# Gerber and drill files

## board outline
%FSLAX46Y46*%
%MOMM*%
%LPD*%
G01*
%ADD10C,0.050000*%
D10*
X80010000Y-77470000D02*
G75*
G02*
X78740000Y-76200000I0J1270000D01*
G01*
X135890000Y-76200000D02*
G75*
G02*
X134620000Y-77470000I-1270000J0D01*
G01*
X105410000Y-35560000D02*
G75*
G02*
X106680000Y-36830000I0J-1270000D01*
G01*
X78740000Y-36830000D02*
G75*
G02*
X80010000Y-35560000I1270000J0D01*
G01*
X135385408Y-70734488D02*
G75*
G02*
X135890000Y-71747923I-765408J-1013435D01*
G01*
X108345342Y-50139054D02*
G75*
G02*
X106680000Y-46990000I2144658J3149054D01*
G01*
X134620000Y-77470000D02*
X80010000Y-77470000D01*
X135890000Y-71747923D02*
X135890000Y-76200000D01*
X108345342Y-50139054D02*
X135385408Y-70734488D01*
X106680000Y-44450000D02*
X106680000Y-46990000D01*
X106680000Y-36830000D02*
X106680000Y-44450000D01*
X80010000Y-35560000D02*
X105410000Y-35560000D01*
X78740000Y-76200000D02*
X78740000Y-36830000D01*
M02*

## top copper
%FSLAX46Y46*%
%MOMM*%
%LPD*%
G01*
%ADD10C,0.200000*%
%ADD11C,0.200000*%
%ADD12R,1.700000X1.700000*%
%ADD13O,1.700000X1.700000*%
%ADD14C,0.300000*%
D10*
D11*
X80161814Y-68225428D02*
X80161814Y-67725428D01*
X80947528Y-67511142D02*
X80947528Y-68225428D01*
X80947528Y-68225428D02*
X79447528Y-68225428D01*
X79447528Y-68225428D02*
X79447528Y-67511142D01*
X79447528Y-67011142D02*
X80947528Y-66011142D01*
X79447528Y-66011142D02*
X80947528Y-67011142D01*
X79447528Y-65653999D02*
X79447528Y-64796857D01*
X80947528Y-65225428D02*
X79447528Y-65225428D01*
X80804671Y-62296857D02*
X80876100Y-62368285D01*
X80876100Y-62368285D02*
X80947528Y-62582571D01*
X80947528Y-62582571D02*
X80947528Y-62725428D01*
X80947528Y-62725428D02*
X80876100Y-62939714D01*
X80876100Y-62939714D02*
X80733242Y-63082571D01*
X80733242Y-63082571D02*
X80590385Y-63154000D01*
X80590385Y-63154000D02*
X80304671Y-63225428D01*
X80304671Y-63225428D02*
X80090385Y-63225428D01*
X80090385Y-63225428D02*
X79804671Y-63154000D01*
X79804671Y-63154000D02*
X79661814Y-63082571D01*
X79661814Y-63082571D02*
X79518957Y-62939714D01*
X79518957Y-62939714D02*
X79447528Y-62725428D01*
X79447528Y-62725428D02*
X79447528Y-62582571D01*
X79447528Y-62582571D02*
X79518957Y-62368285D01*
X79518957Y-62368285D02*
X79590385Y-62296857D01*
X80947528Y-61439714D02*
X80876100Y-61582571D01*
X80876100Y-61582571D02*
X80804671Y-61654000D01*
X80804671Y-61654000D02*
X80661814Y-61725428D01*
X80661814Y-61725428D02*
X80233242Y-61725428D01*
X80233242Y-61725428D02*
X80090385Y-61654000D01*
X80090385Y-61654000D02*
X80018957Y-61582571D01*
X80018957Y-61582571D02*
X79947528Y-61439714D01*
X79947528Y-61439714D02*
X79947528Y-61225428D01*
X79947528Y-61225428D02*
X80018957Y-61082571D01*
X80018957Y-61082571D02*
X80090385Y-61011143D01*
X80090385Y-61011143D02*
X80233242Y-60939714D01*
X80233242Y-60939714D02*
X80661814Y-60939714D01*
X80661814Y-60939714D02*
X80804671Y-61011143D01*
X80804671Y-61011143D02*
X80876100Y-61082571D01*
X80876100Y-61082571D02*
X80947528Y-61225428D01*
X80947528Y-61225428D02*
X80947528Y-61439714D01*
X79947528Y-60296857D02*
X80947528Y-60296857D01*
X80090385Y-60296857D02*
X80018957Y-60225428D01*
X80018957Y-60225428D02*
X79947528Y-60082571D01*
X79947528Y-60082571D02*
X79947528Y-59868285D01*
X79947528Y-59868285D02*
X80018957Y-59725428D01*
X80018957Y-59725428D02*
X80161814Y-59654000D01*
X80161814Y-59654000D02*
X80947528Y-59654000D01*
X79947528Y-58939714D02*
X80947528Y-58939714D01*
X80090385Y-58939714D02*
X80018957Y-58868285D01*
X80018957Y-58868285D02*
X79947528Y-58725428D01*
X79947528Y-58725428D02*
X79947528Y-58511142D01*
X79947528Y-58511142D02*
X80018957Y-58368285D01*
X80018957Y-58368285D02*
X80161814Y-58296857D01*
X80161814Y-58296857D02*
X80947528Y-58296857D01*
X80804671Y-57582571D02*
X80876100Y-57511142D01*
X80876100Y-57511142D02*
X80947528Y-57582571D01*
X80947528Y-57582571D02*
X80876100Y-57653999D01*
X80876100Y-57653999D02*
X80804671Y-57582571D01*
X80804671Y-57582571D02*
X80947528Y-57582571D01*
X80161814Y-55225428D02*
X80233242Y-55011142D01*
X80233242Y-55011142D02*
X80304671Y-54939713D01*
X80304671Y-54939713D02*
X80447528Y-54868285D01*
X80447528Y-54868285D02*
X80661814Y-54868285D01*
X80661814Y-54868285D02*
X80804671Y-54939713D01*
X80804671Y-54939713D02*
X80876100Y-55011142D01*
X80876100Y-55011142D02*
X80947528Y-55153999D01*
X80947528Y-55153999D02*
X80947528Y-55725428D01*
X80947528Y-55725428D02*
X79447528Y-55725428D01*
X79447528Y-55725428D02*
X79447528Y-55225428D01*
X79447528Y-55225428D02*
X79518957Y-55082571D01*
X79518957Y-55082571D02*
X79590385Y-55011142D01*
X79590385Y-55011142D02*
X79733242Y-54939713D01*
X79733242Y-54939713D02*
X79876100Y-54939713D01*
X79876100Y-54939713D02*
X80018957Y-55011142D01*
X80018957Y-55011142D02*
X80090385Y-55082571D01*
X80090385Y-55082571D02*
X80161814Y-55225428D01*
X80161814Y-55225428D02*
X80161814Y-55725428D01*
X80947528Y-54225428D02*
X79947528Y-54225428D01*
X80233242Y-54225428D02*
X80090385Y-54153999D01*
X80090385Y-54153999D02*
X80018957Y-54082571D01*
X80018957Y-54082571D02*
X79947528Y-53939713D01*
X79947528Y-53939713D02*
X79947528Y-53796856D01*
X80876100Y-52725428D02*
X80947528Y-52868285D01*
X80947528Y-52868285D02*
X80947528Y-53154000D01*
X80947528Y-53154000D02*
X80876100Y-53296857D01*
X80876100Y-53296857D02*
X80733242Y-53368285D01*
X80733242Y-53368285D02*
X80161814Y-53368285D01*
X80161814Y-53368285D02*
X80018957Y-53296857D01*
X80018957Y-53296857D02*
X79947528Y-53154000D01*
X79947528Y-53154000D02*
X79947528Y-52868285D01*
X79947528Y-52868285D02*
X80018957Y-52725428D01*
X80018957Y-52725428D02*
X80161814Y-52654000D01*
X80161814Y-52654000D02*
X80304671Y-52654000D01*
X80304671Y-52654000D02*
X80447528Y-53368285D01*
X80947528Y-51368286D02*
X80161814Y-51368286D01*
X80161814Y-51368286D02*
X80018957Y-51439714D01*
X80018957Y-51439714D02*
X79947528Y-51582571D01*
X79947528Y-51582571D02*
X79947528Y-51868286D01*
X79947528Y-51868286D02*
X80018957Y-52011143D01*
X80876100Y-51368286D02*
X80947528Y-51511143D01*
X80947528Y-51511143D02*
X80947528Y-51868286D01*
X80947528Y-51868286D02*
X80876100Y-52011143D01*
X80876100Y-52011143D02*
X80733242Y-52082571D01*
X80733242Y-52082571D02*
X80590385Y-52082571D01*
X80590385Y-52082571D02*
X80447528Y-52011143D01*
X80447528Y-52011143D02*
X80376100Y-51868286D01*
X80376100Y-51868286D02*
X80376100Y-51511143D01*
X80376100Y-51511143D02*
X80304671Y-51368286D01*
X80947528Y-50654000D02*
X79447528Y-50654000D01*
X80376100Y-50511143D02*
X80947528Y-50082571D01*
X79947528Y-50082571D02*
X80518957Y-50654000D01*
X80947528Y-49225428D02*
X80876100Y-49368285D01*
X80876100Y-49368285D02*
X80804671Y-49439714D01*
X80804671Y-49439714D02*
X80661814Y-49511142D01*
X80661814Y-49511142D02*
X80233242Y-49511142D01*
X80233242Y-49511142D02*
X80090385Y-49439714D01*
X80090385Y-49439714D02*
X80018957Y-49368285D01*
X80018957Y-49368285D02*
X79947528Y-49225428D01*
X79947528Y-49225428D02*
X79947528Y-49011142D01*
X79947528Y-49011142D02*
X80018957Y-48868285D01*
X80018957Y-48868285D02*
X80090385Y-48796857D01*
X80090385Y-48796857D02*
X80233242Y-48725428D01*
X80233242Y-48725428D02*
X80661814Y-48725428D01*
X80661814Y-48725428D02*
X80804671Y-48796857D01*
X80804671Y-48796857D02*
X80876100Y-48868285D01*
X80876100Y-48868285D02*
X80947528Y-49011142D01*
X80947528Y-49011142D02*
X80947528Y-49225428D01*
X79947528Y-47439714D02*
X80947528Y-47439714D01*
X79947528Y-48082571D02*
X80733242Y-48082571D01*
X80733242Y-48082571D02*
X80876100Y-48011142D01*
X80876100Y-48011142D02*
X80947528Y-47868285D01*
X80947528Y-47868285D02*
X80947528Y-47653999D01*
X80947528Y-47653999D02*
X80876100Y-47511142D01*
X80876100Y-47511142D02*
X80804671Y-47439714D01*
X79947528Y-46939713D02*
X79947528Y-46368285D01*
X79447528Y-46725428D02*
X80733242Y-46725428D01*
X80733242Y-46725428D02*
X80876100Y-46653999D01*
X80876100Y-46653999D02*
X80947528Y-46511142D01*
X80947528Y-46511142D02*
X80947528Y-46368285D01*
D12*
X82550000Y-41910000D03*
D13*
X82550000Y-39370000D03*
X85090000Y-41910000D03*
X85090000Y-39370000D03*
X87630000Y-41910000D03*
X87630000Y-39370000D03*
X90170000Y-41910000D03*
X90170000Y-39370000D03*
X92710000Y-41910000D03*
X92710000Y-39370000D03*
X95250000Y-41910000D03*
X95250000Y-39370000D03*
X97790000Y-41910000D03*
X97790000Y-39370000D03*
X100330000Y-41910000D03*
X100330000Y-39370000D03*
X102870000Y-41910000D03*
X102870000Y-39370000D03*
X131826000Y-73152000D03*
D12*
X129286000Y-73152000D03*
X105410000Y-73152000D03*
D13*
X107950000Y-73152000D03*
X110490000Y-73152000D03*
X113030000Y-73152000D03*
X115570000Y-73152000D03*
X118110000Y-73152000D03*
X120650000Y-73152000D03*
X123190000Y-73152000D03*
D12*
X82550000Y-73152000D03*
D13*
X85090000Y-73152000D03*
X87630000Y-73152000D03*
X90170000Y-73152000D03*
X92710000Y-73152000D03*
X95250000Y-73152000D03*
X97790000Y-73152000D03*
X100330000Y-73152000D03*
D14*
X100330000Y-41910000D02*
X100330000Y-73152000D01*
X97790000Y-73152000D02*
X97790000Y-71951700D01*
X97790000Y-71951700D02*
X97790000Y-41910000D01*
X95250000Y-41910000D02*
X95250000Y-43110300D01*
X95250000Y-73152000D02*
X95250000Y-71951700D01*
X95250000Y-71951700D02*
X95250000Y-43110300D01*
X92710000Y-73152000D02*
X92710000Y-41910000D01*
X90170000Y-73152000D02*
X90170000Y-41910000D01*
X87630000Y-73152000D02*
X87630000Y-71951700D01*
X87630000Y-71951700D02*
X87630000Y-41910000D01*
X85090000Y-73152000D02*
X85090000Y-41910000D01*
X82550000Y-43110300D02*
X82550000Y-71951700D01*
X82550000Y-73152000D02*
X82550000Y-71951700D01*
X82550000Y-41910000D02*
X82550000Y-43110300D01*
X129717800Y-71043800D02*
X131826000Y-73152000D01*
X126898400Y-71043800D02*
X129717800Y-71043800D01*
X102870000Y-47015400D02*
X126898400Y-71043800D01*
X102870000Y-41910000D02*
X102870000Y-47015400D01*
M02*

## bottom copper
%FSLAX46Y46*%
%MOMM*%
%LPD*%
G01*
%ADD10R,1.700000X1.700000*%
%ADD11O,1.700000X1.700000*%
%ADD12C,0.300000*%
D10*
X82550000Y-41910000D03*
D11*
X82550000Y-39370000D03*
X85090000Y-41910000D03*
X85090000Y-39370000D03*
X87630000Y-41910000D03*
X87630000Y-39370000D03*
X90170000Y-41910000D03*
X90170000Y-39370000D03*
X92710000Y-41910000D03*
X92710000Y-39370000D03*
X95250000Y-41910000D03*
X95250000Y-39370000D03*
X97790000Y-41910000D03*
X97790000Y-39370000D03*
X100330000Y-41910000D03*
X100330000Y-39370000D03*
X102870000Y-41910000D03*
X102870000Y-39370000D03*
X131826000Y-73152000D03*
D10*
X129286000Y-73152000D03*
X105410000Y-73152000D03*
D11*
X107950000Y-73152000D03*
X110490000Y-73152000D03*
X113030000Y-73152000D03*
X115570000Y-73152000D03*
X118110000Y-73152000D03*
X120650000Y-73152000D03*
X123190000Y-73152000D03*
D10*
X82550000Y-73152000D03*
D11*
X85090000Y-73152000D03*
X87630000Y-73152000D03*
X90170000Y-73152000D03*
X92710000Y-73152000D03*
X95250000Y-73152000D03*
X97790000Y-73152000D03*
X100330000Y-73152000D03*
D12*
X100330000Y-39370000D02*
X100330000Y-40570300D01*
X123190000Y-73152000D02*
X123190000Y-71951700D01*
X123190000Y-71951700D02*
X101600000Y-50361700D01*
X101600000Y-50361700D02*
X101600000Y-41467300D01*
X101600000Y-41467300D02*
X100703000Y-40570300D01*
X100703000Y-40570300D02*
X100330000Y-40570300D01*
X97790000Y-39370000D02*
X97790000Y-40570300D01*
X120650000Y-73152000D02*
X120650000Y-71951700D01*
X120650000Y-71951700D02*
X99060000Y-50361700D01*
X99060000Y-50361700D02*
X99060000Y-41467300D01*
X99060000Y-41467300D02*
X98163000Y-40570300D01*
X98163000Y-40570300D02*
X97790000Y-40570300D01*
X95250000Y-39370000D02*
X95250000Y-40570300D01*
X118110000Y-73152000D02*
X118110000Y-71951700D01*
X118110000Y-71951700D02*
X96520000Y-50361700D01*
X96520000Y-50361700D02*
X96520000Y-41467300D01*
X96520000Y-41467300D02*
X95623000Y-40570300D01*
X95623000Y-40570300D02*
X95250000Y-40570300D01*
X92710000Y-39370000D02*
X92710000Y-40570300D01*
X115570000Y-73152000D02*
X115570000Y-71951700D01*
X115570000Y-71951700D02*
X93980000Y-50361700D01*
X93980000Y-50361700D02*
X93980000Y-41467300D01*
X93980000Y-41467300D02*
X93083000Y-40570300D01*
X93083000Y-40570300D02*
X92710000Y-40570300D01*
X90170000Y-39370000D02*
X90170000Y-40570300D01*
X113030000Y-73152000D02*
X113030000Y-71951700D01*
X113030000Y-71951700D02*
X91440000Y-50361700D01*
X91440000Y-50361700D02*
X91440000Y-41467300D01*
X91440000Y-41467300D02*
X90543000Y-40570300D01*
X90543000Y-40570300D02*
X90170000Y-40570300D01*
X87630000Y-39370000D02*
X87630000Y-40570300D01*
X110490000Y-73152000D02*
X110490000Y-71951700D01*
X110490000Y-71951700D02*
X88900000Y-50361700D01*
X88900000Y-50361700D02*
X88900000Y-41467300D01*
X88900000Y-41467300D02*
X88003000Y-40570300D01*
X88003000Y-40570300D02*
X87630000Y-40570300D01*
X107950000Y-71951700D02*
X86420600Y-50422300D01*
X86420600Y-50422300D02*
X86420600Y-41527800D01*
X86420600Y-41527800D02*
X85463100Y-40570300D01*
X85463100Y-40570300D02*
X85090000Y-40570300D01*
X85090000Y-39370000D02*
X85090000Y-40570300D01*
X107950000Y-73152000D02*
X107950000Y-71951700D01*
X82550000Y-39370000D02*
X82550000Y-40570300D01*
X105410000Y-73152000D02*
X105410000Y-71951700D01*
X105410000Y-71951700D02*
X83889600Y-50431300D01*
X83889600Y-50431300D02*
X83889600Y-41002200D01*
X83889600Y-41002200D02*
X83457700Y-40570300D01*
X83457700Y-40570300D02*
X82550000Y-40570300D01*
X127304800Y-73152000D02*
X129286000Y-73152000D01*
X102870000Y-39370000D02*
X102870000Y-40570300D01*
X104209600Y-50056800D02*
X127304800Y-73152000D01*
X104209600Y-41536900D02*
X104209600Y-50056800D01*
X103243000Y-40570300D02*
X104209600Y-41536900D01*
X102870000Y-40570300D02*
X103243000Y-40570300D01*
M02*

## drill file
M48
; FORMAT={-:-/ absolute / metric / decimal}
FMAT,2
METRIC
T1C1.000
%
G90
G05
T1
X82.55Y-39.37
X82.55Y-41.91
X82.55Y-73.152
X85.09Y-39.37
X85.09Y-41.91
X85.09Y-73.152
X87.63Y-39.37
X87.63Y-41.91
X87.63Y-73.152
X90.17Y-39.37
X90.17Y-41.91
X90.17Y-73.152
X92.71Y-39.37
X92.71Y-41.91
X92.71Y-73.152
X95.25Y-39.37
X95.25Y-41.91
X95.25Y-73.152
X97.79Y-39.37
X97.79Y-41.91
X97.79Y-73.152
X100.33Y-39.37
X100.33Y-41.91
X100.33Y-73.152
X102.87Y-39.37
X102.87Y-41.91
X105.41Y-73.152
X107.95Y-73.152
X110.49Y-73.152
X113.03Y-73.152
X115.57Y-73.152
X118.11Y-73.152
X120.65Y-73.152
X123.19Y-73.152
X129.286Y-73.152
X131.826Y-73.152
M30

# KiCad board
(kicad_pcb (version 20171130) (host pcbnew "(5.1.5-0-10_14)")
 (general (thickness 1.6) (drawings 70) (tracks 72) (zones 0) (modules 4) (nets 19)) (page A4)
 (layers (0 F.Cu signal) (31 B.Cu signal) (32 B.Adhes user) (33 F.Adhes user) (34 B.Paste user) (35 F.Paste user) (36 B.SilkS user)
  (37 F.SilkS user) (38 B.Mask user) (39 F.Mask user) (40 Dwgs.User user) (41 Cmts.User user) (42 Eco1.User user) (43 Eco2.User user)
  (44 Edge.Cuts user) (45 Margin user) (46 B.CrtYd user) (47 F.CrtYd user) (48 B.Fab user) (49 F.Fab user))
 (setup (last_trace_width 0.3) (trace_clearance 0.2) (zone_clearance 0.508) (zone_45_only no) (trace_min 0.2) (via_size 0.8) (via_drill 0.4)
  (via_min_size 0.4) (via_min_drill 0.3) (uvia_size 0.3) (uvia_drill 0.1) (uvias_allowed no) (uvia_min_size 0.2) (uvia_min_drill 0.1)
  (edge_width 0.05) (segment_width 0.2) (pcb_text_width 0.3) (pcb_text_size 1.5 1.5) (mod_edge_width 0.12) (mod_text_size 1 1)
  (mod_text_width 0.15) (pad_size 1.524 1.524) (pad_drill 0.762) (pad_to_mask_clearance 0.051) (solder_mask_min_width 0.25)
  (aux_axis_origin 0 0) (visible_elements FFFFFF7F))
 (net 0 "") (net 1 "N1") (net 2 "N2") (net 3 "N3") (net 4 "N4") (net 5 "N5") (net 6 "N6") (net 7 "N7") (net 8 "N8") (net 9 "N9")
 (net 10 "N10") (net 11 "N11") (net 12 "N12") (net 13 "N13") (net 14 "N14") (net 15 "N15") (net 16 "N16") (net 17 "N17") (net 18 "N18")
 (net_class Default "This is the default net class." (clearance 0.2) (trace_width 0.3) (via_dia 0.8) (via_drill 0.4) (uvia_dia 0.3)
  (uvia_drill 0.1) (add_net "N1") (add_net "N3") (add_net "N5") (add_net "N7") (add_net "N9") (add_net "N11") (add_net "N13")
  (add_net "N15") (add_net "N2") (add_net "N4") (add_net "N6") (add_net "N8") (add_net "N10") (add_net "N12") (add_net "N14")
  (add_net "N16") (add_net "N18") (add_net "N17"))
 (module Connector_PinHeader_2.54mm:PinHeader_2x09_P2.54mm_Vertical (layer F.Cu) (at 82.55 41.91 90)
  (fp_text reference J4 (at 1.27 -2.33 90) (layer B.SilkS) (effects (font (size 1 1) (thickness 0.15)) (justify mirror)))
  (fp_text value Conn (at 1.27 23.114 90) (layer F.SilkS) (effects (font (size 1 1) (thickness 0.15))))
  (pad 1 thru_hole rect (at 0 0 90) (size 1.7 1.7) (drill 1) (layers *.Cu *.Mask) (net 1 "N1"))
  (pad 2 thru_hole oval (at 2.54 0 90) (size 1.7 1.7) (drill 1) (layers *.Cu *.Mask) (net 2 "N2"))
  (pad 3 thru_hole oval (at 0 2.54 90) (size 1.7 1.7) (drill 1) (layers *.Cu *.Mask) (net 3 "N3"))
  (pad 4 thru_hole oval (at 2.54 2.54 90) (size 1.7 1.7) (drill 1) (layers *.Cu *.Mask) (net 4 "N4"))
  (pad 5 thru_hole oval (at 0 5.08 90) (size 1.7 1.7) (drill 1) (layers *.Cu *.Mask) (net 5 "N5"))
  (pad 6 thru_hole oval (at 2.54 5.08 90) (size 1.7 1.7) (drill 1) (layers *.Cu *.Mask) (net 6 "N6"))
  (pad 7 thru_hole oval (at 0 7.62 90) (size 1.7 1.7) (drill 1) (layers *.Cu *.Mask) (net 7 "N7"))
  (pad 8 thru_hole oval (at 2.54 7.62 90) (size 1.7 1.7) (drill 1) (layers *.Cu *.Mask) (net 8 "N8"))
  (pad 9 thru_hole oval (at 0 10.16 90) (size 1.7 1.7) (drill 1) (layers *.Cu *.Mask) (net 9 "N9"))
  (pad 10 thru_hole oval (at 2.54 10.16 90) (size 1.7 1.7) (drill 1) (layers *.Cu *.Mask) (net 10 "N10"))
  (pad 11 thru_hole oval (at 0 12.7 90) (size 1.7 1.7) (drill 1) (layers *.Cu *.Mask) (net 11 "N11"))
  (pad 12 thru_hole oval (at 2.54 12.7 90) (size 1.7 1.7) (drill 1) (layers *.Cu *.Mask) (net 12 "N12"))
  (pad 13 thru_hole oval (at 0 15.24 90) (size 1.7 1.7) (drill 1) (layers *.Cu *.Mask) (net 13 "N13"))
  (pad 14 thru_hole oval (at 2.54 15.24 90) (size 1.7 1.7) (drill 1) (layers *.Cu *.Mask) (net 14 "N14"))
  (pad 15 thru_hole oval (at 0 17.78 90) (size 1.7 1.7) (drill 1) (layers *.Cu *.Mask) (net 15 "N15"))
  (pad 16 thru_hole oval (at 2.54 17.78 90) (size 1.7 1.7) (drill 1) (layers *.Cu *.Mask) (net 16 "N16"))
  (pad 17 thru_hole oval (at 0 20.32 90) (size 1.7 1.7) (drill 1) (layers *.Cu *.Mask) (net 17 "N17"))
  (pad 18 thru_hole oval (at 2.54 20.32 90) (size 1.7 1.7) (drill 1) (layers *.Cu *.Mask) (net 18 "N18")))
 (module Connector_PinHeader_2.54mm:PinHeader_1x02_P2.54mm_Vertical (layer B.Cu) (at 129.286 73.152 270)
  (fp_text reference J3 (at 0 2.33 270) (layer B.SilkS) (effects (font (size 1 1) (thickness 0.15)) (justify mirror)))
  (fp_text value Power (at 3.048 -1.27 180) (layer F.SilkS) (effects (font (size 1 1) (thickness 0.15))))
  (pad 2 thru_hole oval (at 0 -2.54 270) (size 1.7 1.7) (drill 1) (layers *.Cu *.Mask) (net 17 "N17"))
  (pad 1 thru_hole rect (at 0 0 270) (size 1.7 1.7) (drill 1) (layers *.Cu *.Mask) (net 18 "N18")))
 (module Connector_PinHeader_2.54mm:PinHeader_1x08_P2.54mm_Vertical (layer B.Cu) (at 105.41 73.152 270)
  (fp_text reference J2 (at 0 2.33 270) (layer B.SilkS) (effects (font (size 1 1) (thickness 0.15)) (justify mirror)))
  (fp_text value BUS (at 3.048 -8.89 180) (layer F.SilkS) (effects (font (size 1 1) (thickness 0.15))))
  (pad 1 thru_hole rect (at 0 0 270) (size 1.7 1.7) (drill 1) (layers *.Cu *.Mask) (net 2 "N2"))
  (pad 2 thru_hole oval (at 0 -2.54 270) (size 1.7 1.7) (drill 1) (layers *.Cu *.Mask) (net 4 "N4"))
  (pad 3 thru_hole oval (at 0 -5.08 270) (size 1.7 1.7) (drill 1) (layers *.Cu *.Mask) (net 6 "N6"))
  (pad 4 thru_hole oval (at 0 -7.62 270) (size 1.7 1.7) (drill 1) (layers *.Cu *.Mask) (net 8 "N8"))
  (pad 5 thru_hole oval (at 0 -10.16 270) (size 1.7 1.7) (drill 1) (layers *.Cu *.Mask) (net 10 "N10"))
  (pad 6 thru_hole oval (at 0 -12.7 270) (size 1.7 1.7) (drill 1) (layers *.Cu *.Mask) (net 12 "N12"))
  (pad 7 thru_hole oval (at 0 -15.24 270) (size 1.7 1.7) (drill 1) (layers *.Cu *.Mask) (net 14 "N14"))
  (pad 8 thru_hole oval (at 0 -17.78 270) (size 1.7 1.7) (drill 1) (layers *.Cu *.Mask) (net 16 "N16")))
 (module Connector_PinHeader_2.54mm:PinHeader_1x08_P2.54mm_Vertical (layer B.Cu) (at 82.55 73.152 270)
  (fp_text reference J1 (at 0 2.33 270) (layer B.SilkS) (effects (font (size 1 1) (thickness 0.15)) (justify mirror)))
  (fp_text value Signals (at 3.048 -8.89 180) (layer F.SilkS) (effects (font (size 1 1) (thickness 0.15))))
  (pad 1 thru_hole rect (at 0 0 270) (size 1.7 1.7) (drill 1) (layers *.Cu *.Mask) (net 1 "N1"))
  (pad 2 thru_hole oval (at 0 -2.54 270) (size 1.7 1.7) (drill 1) (layers *.Cu *.Mask) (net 3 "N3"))
  (pad 3 thru_hole oval (at 0 -5.08 270) (size 1.7 1.7) (drill 1) (layers *.Cu *.Mask) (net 5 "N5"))
  (pad 4 thru_hole oval (at 0 -7.62 270) (size 1.7 1.7) (drill 1) (layers *.Cu *.Mask) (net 7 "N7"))
  (pad 5 thru_hole oval (at 0 -10.16 270) (size 1.7 1.7) (drill 1) (layers *.Cu *.Mask) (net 9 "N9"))
  (pad 6 thru_hole oval (at 0 -12.7 270) (size 1.7 1.7) (drill 1) (layers *.Cu *.Mask) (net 11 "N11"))
  (pad 7 thru_hole oval (at 0 -15.24 270) (size 1.7 1.7) (drill 1) (layers *.Cu *.Mask) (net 13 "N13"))
  (pad 8 thru_hole oval (at 0 -17.78 270) (size 1.7 1.7) (drill 1) (layers *.Cu *.Mask) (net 15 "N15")))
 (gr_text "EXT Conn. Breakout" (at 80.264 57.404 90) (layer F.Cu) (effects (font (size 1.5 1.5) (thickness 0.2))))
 (gr_arc (start 80.01 76.2) (end 78.74 76.2) (angle -90) (layer Edge.Cuts) (width 0.05))
 (gr_arc (start 134.62 76.2) (end 134.62 77.47) (angle -90) (layer Edge.Cuts) (width 0.05))
 (gr_arc (start 105.41 36.83) (end 106.68 36.83) (angle -90) (layer Edge.Cuts) (width 0.05))
 (gr_arc (start 80.01 36.83) (end 80.01 35.56) (angle -90) (layer Edge.Cuts) (width 0.05))
 (gr_arc (start 134.62 71.747923) (end 135.89 71.747923) (angle -52.93767885) (layer Edge.Cuts) (width 0.05))
 (gr_arc (start 110.49 46.99) (end 106.68 46.99) (angle -55.74323869) (layer Edge.Cuts) (width 0.05))
 (gr_line (start 134.62 77.47) (end 80.01 77.47) (layer Edge.Cuts) (width 0.05))
 (gr_line (start 135.89 71.747923) (end 135.89 76.2) (layer Edge.Cuts) (width 0.05))
 (gr_line (start 108.345342 50.139054) (end 135.385408 70.734488) (layer Edge.Cuts) (width 0.05))
 (gr_line (start 106.68 44.45) (end 106.68 46.99) (layer Edge.Cuts) (width 0.05))
 (gr_line (start 106.68 36.83) (end 106.68 44.45) (layer Edge.Cuts) (width 0.05))
 (gr_line (start 80.01 35.56) (end 105.41 35.56) (layer Edge.Cuts) (width 0.05))
 (gr_line (start 78.74 76.2) (end 78.74 36.83) (layer Edge.Cuts) (width 0.05))
 (segment (start 100.33 41.91) (end 100.33 73.152) (width 0.3) (layer F.Cu) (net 15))
 (segment (start 97.79 73.152) (end 97.79 71.9517) (width 0.3) (layer F.Cu) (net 13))
 (segment (start 97.79 71.9517) (end 97.79 41.91) (width 0.3) (layer F.Cu) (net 13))
 (segment (start 95.25 41.91) (end 95.25 43.1103) (width 0.3) (layer F.Cu) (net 11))
 (segment (start 95.25 73.152) (end 95.25 71.9517) (width 0.3) (layer F.Cu) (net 11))
 (segment (start 95.25 71.9517) (end 95.25 43.1103) (width 0.3) (layer F.Cu) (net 11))
 (segment (start 92.71 73.152) (end 92.71 41.91) (width 0.3) (layer F.Cu) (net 9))
 (segment (start 90.17 73.152) (end 90.17 41.91) (width 0.3) (layer F.Cu) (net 7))
 (segment (start 87.63 73.152) (end 87.63 71.9517) (width 0.3) (layer F.Cu) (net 5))
 (segment (start 87.63 71.9517) (end 87.63 41.91) (width 0.3) (layer F.Cu) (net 5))
 (segment (start 85.09 73.152) (end 85.09 41.91) (width 0.3) (layer F.Cu) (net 3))
 (segment (start 82.55 43.1103) (end 82.55 71.9517) (width 0.3) (layer F.Cu) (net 1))
 (segment (start 82.55 73.152) (end 82.55 71.9517) (width 0.3) (layer F.Cu) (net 1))
 (segment (start 82.55 41.91) (end 82.55 43.1103) (width 0.3) (layer F.Cu) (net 1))
 (segment (start 100.33 39.37) (end 100.33 40.5703) (width 0.3) (layer B.Cu) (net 16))
 (segment (start 123.19 73.152) (end 123.19 71.9517) (width 0.3) (layer B.Cu) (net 16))
 (segment (start 123.19 71.9517) (end 101.6 50.3617) (width 0.3) (layer B.Cu) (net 16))
 (segment (start 101.6 50.3617) (end 101.6 41.4673) (width 0.3) (layer B.Cu) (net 16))
 (segment (start 101.6 41.4673) (end 100.703 40.5703) (width 0.3) (layer B.Cu) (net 16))
 (segment (start 100.703 40.5703) (end 100.33 40.5703) (width 0.3) (layer B.Cu) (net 16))
 (segment (start 97.79 39.37) (end 97.79 40.5703) (width 0.3) (layer B.Cu) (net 14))
 (segment (start 120.65 73.152) (end 120.65 71.9517) (width 0.3) (layer B.Cu) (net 14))
 (segment (start 120.65 71.9517) (end 99.06 50.3617) (width 0.3) (layer B.Cu) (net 14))
 (segment (start 99.06 50.3617) (end 99.06 41.4673) (width 0.3) (layer B.Cu) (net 14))
 (segment (start 99.06 41.4673) (end 98.163 40.5703) (width 0.3) (layer B.Cu) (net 14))
 (segment (start 98.163 40.5703) (end 97.79 40.5703) (width 0.3) (layer B.Cu) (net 14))
 (segment (start 95.25 39.37) (end 95.25 40.5703) (width 0.3) (layer B.Cu) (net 12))
 (segment (start 118.11 73.152) (end 118.11 71.9517) (width 0.3) (layer B.Cu) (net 12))
 (segment (start 118.11 71.9517) (end 96.52 50.3617) (width 0.3) (layer B.Cu) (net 12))
 (segment (start 96.52 50.3617) (end 96.52 41.4673) (width 0.3) (layer B.Cu) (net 12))
 (segment (start 96.52 41.4673) (end 95.623 40.5703) (width 0.3) (layer B.Cu) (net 12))
 (segment (start 95.623 40.5703) (end 95.25 40.5703) (width 0.3) (layer B.Cu) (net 12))
 (segment (start 92.71 39.37) (end 92.71 40.5703) (width 0.3) (layer B.Cu) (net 10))
 (segment (start 115.57 73.152) (end 115.57 71.9517) (width 0.3) (layer B.Cu) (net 10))
 (segment (start 115.57 71.9517) (end 93.98 50.3617) (width 0.3) (layer B.Cu) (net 10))
 (segment (start 93.98 50.3617) (end 93.98 41.4673) (width 0.3) (layer B.Cu) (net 10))
 (segment (start 93.98 41.4673) (end 93.083 40.5703) (width 0.3) (layer B.Cu) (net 10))
 (segment (start 93.083 40.5703) (end 92.71 40.5703) (width 0.3) (layer B.Cu) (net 10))
 (segment (start 90.17 39.37) (end 90.17 40.5703) (width 0.3) (layer B.Cu) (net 8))
 (segment (start 113.03 73.152) (end 113.03 71.9517) (width 0.3) (layer B.Cu) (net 8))
 (segment (start 113.03 71.9517) (end 91.44 50.3617) (width 0.3) (layer B.Cu) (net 8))
 (segment (start 91.44 50.3617) (end 91.44 41.4673) (width 0.3) (layer B.Cu) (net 8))
 (segment (start 91.44 41.4673) (end 90.543 40.5703) (width 0.3) (layer B.Cu) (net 8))
 (segment (start 90.543 40.5703) (end 90.17 40.5703) (width 0.3) (layer B.Cu) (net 8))
 (segment (start 87.63 39.37) (end 87.63 40.5703) (width 0.3) (layer B.Cu) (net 6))
 (segment (start 110.49 73.152) (end 110.49 71.9517) (width 0.3) (layer B.Cu) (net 6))
 (segment (start 110.49 71.9517) (end 88.9 50.3617) (width 0.3) (layer B.Cu) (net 6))
 (segment (start 88.9 50.3617) (end 88.9 41.4673) (width 0.3) (layer B.Cu) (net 6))
 (segment (start 88.9 41.4673) (end 88.003 40.5703) (width 0.3) (layer B.Cu) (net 6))
 (segment (start 88.003 40.5703) (end 87.63 40.5703) (width 0.3) (layer B.Cu) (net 6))
 (segment (start 107.95 71.9517) (end 86.4206 50.4223) (width 0.3) (layer B.Cu) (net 4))
 (segment (start 86.4206 50.4223) (end 86.4206 41.5278) (width 0.3) (layer B.Cu) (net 4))
 (segment (start 86.4206 41.5278) (end 85.4631 40.5703) (width 0.3) (layer B.Cu) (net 4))
 (segment (start 85.4631 40.5703) (end 85.09 40.5703) (width 0.3) (layer B.Cu) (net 4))
 (segment (start 85.09 39.37) (end 85.09 40.5703) (width 0.3) (layer B.Cu) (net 4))
 (segment (start 107.95 73.152) (end 107.95 71.9517) (width 0.3) (layer B.Cu) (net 4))
 (segment (start 82.55 39.37) (end 82.55 40.5703) (width 0.3) (layer B.Cu) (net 2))
 (segment (start 105.41 73.152) (end 105.41 71.9517) (width 0.3) (layer B.Cu) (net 2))
 (segment (start 105.41 71.9517) (end 83.8896 50.4313) (width 0.3) (layer B.Cu) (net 2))
 (segment (start 83.8896 50.4313) (end 83.8896 41.0022) (width 0.3) (layer B.Cu) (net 2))
 (segment (start 83.8896 41.0022) (end 83.4577 40.5703) (width 0.3) (layer B.Cu) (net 2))
 (segment (start 83.4577 40.5703) (end 82.55 40.5703) (width 0.3) (layer B.Cu) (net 2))
 (segment (start 129.7178 71.0438) (end 131.826 73.152) (width 0.3) (layer F.Cu) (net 17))
 (segment (start 126.8984 71.0438) (end 129.7178 71.0438) (width 0.3) (layer F.Cu) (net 17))
 (segment (start 102.87 47.0154) (end 126.8984 71.0438) (width 0.3) (layer F.Cu) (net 17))
 (segment (start 102.87 41.91) (end 102.87 47.0154) (width 0.3) (layer F.Cu) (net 17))
 (segment (start 127.3048 73.152) (end 129.286 73.152) (width 0.3) (layer B.Cu) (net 18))
 (segment (start 102.87 39.37) (end 102.87 40.5703) (width 0.3) (layer B.Cu) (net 18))
 (segment (start 104.2096 50.0568) (end 127.3048 73.152) (width 0.3) (layer B.Cu) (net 18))
 (segment (start 104.2096 41.5369) (end 104.2096 50.0568) (width 0.3) (layer B.Cu) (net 18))
 (segment (start 103.243 40.5703) (end 104.2096 41.5369) (width 0.3) (layer B.Cu) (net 18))
 (segment (start 102.87 40.5703) (end 103.243 40.5703) (width 0.3) (layer B.Cu) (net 18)))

